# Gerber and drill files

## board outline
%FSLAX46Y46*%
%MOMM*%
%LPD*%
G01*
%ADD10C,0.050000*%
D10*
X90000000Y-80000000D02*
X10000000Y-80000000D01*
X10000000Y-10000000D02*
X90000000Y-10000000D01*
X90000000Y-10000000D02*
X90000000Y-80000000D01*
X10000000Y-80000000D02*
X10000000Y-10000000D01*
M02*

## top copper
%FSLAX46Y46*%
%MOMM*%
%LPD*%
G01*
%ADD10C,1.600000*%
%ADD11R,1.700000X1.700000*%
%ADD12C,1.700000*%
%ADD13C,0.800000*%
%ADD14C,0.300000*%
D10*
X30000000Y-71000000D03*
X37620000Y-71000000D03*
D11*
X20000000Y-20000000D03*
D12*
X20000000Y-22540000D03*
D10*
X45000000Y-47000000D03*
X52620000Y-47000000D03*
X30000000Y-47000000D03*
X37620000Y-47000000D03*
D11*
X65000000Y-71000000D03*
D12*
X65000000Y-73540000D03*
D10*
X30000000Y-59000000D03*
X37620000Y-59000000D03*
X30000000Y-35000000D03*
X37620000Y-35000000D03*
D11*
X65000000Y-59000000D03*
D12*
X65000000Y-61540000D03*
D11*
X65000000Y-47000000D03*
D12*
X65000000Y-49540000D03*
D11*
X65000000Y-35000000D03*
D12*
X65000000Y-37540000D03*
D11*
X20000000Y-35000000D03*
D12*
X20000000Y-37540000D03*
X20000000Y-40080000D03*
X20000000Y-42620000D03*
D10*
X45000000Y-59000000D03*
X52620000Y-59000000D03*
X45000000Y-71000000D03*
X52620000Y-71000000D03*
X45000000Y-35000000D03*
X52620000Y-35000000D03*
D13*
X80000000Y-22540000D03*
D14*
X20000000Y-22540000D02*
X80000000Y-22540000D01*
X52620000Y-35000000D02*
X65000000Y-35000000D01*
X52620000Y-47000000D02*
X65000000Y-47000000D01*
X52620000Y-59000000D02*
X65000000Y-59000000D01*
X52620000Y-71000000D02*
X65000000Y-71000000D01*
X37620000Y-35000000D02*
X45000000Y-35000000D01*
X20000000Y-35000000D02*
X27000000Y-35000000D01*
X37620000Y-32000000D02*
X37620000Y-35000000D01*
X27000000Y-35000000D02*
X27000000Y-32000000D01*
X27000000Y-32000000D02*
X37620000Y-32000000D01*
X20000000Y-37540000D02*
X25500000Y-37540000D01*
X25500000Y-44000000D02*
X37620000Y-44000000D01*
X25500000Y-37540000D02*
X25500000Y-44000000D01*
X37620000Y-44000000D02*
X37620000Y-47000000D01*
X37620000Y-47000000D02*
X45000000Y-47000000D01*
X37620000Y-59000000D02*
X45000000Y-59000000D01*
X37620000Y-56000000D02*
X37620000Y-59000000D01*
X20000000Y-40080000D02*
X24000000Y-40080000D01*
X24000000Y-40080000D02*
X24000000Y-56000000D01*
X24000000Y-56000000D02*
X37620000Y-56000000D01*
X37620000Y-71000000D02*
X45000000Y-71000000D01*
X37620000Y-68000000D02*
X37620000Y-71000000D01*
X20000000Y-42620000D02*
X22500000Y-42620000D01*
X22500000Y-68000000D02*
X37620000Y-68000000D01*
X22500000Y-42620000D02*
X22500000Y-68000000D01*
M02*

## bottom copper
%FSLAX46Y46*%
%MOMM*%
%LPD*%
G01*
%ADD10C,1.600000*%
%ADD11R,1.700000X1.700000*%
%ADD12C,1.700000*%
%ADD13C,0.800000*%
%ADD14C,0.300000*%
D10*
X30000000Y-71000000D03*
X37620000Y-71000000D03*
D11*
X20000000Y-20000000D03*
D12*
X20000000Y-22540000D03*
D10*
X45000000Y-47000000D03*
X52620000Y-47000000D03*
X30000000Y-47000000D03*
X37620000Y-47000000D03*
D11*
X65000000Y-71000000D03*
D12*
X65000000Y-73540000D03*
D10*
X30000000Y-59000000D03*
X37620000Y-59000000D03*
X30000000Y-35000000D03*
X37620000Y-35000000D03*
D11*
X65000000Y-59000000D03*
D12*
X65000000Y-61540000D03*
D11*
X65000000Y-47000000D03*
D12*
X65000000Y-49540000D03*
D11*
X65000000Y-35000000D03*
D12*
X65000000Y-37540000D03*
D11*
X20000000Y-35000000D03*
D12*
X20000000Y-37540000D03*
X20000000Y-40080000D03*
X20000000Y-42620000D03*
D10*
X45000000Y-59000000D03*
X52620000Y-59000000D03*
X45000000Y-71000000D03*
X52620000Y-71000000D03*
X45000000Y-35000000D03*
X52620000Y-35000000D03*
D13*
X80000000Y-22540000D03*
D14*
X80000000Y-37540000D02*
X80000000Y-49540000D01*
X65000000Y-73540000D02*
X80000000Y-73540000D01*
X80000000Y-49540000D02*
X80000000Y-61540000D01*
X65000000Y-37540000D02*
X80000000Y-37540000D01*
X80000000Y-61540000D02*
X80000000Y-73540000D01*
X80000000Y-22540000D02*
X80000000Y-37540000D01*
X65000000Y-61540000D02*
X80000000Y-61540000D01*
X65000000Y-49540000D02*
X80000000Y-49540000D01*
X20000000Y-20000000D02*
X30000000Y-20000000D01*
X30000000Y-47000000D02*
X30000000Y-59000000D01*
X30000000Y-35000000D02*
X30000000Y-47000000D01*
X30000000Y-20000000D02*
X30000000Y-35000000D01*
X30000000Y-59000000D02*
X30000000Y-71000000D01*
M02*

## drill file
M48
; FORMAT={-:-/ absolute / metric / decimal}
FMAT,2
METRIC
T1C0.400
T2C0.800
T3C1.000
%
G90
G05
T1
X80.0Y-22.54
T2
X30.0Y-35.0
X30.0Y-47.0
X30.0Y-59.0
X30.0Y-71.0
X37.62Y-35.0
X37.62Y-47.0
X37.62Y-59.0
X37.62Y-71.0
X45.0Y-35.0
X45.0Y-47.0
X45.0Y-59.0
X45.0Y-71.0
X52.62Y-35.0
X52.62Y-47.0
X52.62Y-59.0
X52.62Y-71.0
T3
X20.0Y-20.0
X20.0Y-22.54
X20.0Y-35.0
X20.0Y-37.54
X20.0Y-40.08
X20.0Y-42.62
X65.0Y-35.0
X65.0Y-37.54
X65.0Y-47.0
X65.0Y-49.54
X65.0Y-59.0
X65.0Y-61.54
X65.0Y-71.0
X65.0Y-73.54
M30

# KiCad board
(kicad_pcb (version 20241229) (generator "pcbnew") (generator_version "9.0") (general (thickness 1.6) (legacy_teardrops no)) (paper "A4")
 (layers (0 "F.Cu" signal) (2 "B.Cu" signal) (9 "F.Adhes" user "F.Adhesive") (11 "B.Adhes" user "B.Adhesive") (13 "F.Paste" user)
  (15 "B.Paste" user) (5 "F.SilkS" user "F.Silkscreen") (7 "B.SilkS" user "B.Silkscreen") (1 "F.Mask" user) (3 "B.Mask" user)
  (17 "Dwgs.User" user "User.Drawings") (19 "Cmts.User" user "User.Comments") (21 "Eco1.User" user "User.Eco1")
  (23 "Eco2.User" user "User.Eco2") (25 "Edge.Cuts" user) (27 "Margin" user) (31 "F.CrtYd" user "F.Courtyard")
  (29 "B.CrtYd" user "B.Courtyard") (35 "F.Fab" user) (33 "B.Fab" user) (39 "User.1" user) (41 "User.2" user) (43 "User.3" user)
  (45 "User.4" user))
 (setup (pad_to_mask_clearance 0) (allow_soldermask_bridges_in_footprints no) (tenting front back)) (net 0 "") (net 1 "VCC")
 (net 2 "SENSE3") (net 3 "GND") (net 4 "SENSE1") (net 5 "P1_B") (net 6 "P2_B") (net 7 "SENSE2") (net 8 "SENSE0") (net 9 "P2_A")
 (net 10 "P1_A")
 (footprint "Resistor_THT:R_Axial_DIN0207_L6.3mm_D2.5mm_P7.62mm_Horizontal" (layer "F.Cu") (at 30 71)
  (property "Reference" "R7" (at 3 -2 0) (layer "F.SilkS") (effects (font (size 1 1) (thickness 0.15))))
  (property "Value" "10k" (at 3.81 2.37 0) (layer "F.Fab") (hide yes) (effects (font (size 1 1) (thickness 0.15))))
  (pad "1" thru_hole circle (at 0 0) (size 1.6 1.6) (drill 0.8) (layers "*.Cu" "*.Mask") (remove_unused_layers no) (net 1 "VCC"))
  (pad "2" thru_hole circle (at 7.62 0) (size 1.6 1.6) (drill 0.8) (layers "*.Cu" "*.Mask") (remove_unused_layers no) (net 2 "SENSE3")))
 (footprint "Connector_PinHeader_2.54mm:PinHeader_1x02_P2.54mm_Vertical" (layer "F.Cu") (at 20 20)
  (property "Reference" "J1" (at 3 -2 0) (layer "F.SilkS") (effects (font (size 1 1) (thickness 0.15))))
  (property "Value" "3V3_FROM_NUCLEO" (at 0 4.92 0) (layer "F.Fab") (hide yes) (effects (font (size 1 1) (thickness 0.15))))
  (pad "1" thru_hole rect (at 0 0) (size 1.7 1.7) (drill 1) (layers "*.Cu" "*.Mask") (remove_unused_layers no) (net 1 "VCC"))
  (pad "2" thru_hole circle (at 0 2.54) (size 1.7 1.7) (drill 1) (layers "*.Cu" "*.Mask") (remove_unused_layers no) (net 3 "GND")))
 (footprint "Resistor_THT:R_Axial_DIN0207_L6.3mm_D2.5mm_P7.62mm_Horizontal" (layer "F.Cu") (at 45 47)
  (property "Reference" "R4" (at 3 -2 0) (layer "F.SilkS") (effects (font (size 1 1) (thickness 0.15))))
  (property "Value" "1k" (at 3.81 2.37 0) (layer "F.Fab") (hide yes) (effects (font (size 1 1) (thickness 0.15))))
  (pad "1" thru_hole circle (at 0 0) (size 1.6 1.6) (drill 0.8) (layers "*.Cu" "*.Mask") (remove_unused_layers no) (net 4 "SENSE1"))
  (pad "2" thru_hole circle (at 7.62 0) (size 1.6 1.6) (drill 0.8) (layers "*.Cu" "*.Mask") (remove_unused_layers no) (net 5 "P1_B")))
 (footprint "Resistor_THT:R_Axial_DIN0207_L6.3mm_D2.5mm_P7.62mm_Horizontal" (layer "F.Cu") (at 30 47)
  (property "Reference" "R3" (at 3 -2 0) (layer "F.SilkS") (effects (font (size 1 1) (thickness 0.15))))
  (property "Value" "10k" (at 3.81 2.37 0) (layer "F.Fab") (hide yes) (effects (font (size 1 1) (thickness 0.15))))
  (pad "1" thru_hole circle (at 0 0) (size 1.6 1.6) (drill 0.8) (layers "*.Cu" "*.Mask") (remove_unused_layers no) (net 1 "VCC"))
  (pad "2" thru_hole circle (at 7.62 0) (size 1.6 1.6) (drill 0.8) (layers "*.Cu" "*.Mask") (remove_unused_layers no) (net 4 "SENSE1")))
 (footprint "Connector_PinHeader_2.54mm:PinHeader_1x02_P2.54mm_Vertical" (layer "F.Cu") (at 65 71)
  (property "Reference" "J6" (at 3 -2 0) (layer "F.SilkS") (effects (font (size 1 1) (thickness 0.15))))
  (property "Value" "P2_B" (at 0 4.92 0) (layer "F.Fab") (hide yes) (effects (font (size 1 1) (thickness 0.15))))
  (pad "1" thru_hole rect (at 0 0) (size 1.7 1.7) (drill 1) (layers "*.Cu" "*.Mask") (remove_unused_layers no) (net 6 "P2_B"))
  (pad "2" thru_hole circle (at 0 2.54) (size 1.7 1.7) (drill 1) (layers "*.Cu" "*.Mask") (remove_unused_layers no) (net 3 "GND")))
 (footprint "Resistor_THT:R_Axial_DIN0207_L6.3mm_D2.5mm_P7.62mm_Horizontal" (layer "F.Cu") (at 30 59)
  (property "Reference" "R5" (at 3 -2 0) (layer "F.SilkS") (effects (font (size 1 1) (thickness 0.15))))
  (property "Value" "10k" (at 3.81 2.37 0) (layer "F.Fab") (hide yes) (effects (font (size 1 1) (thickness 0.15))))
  (pad "1" thru_hole circle (at 0 0) (size 1.6 1.6) (drill 0.8) (layers "*.Cu" "*.Mask") (remove_unused_layers no) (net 1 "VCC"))
  (pad "2" thru_hole circle (at 7.62 0) (size 1.6 1.6) (drill 0.8) (layers "*.Cu" "*.Mask") (remove_unused_layers no) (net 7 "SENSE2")))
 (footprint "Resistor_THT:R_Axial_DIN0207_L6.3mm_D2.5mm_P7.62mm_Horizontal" (layer "F.Cu") (at 30 35)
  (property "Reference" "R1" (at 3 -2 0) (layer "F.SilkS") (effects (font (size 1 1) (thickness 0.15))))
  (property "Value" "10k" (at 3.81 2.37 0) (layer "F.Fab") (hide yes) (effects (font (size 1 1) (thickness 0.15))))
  (pad "1" thru_hole circle (at 0 0) (size 1.6 1.6) (drill 0.8) (layers "*.Cu" "*.Mask") (remove_unused_layers no) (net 1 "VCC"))
  (pad "2" thru_hole circle (at 7.62 0) (size 1.6 1.6) (drill 0.8) (layers "*.Cu" "*.Mask") (remove_unused_layers no) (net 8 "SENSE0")))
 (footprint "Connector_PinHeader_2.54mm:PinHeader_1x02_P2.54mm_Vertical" (layer "F.Cu") (at 65 59)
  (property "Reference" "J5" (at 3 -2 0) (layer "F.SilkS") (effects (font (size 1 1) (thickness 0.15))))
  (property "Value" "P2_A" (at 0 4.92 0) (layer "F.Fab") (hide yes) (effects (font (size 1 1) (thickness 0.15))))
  (pad "1" thru_hole rect (at 0 0) (size 1.7 1.7) (drill 1) (layers "*.Cu" "*.Mask") (remove_unused_layers no) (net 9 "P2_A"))
  (pad "2" thru_hole circle (at 0 2.54) (size 1.7 1.7) (drill 1) (layers "*.Cu" "*.Mask") (remove_unused_layers no) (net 3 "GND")))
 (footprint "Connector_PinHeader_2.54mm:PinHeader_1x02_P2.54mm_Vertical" (layer "F.Cu") (at 65 47)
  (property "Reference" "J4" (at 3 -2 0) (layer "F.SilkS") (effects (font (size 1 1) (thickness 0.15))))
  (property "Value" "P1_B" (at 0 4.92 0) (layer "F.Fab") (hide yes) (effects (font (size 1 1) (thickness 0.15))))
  (pad "1" thru_hole rect (at 0 0) (size 1.7 1.7) (drill 1) (layers "*.Cu" "*.Mask") (remove_unused_layers no) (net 5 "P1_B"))
  (pad "2" thru_hole circle (at 0 2.54) (size 1.7 1.7) (drill 1) (layers "*.Cu" "*.Mask") (remove_unused_layers no) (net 3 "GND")))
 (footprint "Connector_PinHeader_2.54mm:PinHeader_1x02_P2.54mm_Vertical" (layer "F.Cu") (at 65 35)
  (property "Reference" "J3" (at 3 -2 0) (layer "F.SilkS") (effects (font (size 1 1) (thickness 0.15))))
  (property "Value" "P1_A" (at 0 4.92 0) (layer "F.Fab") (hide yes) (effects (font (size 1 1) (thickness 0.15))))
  (pad "1" thru_hole rect (at 0 0) (size 1.7 1.7) (drill 1) (layers "*.Cu" "*.Mask") (remove_unused_layers no) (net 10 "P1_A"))
  (pad "2" thru_hole circle (at 0 2.54) (size 1.7 1.7) (drill 1) (layers "*.Cu" "*.Mask") (remove_unused_layers no) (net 3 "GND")))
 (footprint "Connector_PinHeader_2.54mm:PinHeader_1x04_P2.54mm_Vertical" (layer "F.Cu") (at 20 35)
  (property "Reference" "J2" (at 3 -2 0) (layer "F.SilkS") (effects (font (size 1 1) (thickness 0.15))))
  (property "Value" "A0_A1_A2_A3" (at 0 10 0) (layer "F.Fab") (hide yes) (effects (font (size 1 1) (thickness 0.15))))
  (pad "1" thru_hole rect (at 0 0) (size 1.7 1.7) (drill 1) (layers "*.Cu" "*.Mask") (remove_unused_layers no) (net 8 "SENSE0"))
  (pad "2" thru_hole circle (at 0 2.54) (size 1.7 1.7) (drill 1) (layers "*.Cu" "*.Mask") (remove_unused_layers no) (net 4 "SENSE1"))
  (pad "3" thru_hole circle (at 0 5.08) (size 1.7 1.7) (drill 1) (layers "*.Cu" "*.Mask") (remove_unused_layers no) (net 7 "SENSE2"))
  (pad "4" thru_hole circle (at 0 7.62) (size 1.7 1.7) (drill 1) (layers "*.Cu" "*.Mask") (remove_unused_layers no) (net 2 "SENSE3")))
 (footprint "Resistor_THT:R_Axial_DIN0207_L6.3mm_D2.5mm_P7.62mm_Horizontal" (layer "F.Cu") (at 45 59)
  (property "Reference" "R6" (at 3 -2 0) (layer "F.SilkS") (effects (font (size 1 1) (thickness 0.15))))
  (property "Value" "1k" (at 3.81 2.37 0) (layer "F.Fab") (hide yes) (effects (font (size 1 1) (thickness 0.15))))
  (pad "1" thru_hole circle (at 0 0) (size 1.6 1.6) (drill 0.8) (layers "*.Cu" "*.Mask") (remove_unused_layers no) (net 7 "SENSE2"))
  (pad "2" thru_hole circle (at 7.62 0) (size 1.6 1.6) (drill 0.8) (layers "*.Cu" "*.Mask") (remove_unused_layers no) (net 9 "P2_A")))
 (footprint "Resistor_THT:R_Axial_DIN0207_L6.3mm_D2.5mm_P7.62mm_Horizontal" (layer "F.Cu") (at 45 71)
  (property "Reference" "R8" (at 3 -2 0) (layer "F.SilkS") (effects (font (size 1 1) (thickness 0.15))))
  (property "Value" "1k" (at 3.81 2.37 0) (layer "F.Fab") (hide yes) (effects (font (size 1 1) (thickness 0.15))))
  (pad "1" thru_hole circle (at 0 0) (size 1.6 1.6) (drill 0.8) (layers "*.Cu" "*.Mask") (remove_unused_layers no) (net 2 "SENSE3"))
  (pad "2" thru_hole circle (at 7.62 0) (size 1.6 1.6) (drill 0.8) (layers "*.Cu" "*.Mask") (remove_unused_layers no) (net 6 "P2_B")))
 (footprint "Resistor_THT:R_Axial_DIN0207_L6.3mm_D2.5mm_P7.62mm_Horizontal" (layer "F.Cu") (at 45 35)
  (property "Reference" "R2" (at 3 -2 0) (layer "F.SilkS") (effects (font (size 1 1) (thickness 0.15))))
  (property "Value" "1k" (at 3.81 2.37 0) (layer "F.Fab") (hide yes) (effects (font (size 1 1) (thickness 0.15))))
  (pad "1" thru_hole circle (at 0 0) (size 1.6 1.6) (drill 0.8) (layers "*.Cu" "*.Mask") (remove_unused_layers no) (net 8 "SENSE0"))
  (pad "2" thru_hole circle (at 7.62 0) (size 1.6 1.6) (drill 0.8) (layers "*.Cu" "*.Mask") (remove_unused_layers no) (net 10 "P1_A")))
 (gr_line (start 90 80) (end 10 80) (stroke (width 0.05) (type default)) (layer "Edge.Cuts"))
 (gr_line (start 10 10) (end 90 10) (stroke (width 0.05) (type default)) (layer "Edge.Cuts"))
 (gr_line (start 90 10) (end 90 80) (stroke (width 0.05) (type default)) (layer "Edge.Cuts"))
 (gr_line (start 10 80) (end 10 10) (stroke (width 0.05) (type default)) (layer "Edge.Cuts"))
 (segment (start 20 22.54) (end 80 22.54) (width 0.3) (layer "F.Cu") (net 3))
 (via (at 80 22.54) (size 0.8) (drill 0.4) (layers "F.Cu" "B.Cu") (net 3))
 (segment (start 80 37.54) (end 80 49.54) (width 0.3) (layer "B.Cu") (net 3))
 (segment (start 65 73.54) (end 80 73.54) (width 0.3) (layer "B.Cu") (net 3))
 (segment (start 80 49.54) (end 80 61.54) (width 0.3) (layer "B.Cu") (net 3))
 (segment (start 65 37.54) (end 80 37.54) (width 0.3) (layer "B.Cu") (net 3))
 (segment (start 80 61.54) (end 80 73.54) (width 0.3) (layer "B.Cu") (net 3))
 (segment (start 80 22.54) (end 80 37.54) (width 0.3) (layer "B.Cu") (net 3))
 (segment (start 65 61.54) (end 80 61.54) (width 0.3) (layer "B.Cu") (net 3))
 (segment (start 65 49.54) (end 80 49.54) (width 0.3) (layer "B.Cu") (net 3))
 (segment (start 52.62 35) (end 65 35) (width 0.3) (layer "F.Cu") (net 10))
 (segment (start 52.62 47) (end 65 47) (width 0.3) (layer "F.Cu") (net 5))
 (segment (start 52.62 59) (end 65 59) (width 0.3) (layer "F.Cu") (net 9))
 (segment (start 52.62 71) (end 65 71) (width 0.3) (layer "F.Cu") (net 6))
 (segment (start 37.62 35) (end 45 35) (width 0.3) (layer "F.Cu") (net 8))
 (segment (start 20 35) (end 27 35) (width 0.3) (layer "F.Cu") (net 8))
 (segment (start 37.62 32) (end 37.62 35) (width 0.3) (layer "F.Cu") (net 8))
 (segment (start 27 35) (end 27 32) (width 0.3) (layer "F.Cu") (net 8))
 (segment (start 27 32) (end 37.62 32) (width 0.3) (layer "F.Cu") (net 8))
 (segment (start 20 37.54) (end 25.5 37.54) (width 0.3) (layer "F.Cu") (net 4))
 (segment (start 25.5 44) (end 37.62 44) (width 0.3) (layer "F.Cu") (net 4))
 (segment (start 25.5 37.54) (end 25.5 44) (width 0.3) (layer "F.Cu") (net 4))
 (segment (start 37.62 44) (end 37.62 47) (width 0.3) (layer "F.Cu") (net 4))
 (segment (start 37.62 47) (end 45 47) (width 0.3) (layer "F.Cu") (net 4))
 (segment (start 37.62 59) (end 45 59) (width 0.3) (layer "F.Cu") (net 7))
 (segment (start 37.62 56) (end 37.62 59) (width 0.3) (layer "F.Cu") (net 7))
 (segment (start 20 40.08) (end 24 40.08) (width 0.3) (layer "F.Cu") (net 7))
 (segment (start 24 40.08) (end 24 56) (width 0.3) (layer "F.Cu") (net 7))
 (segment (start 24 56) (end 37.62 56) (width 0.3) (layer "F.Cu") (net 7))
 (segment (start 37.62 71) (end 45 71) (width 0.3) (layer "F.Cu") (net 2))
 (segment (start 37.62 68) (end 37.62 71) (width 0.3) (layer "F.Cu") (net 2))
 (segment (start 20 42.62) (end 22.5 42.62) (width 0.3) (layer "F.Cu") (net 2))
 (segment (start 22.5 68) (end 37.62 68) (width 0.3) (layer "F.Cu") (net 2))
 (segment (start 22.5 42.62) (end 22.5 68) (width 0.3) (layer "F.Cu") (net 2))
 (segment (start 20 20) (end 30 20) (width 0.3) (layer "B.Cu") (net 1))
 (segment (start 30 47) (end 30 59) (width 0.3) (layer "B.Cu") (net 1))
 (segment (start 30 35) (end 30 47) (width 0.3) (layer "B.Cu") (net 1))
 (segment (start 30 20) (end 30 35) (width 0.3) (layer "B.Cu") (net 1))
 (segment (start 30 59) (end 30 71) (width 0.3) (layer "B.Cu") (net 1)))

